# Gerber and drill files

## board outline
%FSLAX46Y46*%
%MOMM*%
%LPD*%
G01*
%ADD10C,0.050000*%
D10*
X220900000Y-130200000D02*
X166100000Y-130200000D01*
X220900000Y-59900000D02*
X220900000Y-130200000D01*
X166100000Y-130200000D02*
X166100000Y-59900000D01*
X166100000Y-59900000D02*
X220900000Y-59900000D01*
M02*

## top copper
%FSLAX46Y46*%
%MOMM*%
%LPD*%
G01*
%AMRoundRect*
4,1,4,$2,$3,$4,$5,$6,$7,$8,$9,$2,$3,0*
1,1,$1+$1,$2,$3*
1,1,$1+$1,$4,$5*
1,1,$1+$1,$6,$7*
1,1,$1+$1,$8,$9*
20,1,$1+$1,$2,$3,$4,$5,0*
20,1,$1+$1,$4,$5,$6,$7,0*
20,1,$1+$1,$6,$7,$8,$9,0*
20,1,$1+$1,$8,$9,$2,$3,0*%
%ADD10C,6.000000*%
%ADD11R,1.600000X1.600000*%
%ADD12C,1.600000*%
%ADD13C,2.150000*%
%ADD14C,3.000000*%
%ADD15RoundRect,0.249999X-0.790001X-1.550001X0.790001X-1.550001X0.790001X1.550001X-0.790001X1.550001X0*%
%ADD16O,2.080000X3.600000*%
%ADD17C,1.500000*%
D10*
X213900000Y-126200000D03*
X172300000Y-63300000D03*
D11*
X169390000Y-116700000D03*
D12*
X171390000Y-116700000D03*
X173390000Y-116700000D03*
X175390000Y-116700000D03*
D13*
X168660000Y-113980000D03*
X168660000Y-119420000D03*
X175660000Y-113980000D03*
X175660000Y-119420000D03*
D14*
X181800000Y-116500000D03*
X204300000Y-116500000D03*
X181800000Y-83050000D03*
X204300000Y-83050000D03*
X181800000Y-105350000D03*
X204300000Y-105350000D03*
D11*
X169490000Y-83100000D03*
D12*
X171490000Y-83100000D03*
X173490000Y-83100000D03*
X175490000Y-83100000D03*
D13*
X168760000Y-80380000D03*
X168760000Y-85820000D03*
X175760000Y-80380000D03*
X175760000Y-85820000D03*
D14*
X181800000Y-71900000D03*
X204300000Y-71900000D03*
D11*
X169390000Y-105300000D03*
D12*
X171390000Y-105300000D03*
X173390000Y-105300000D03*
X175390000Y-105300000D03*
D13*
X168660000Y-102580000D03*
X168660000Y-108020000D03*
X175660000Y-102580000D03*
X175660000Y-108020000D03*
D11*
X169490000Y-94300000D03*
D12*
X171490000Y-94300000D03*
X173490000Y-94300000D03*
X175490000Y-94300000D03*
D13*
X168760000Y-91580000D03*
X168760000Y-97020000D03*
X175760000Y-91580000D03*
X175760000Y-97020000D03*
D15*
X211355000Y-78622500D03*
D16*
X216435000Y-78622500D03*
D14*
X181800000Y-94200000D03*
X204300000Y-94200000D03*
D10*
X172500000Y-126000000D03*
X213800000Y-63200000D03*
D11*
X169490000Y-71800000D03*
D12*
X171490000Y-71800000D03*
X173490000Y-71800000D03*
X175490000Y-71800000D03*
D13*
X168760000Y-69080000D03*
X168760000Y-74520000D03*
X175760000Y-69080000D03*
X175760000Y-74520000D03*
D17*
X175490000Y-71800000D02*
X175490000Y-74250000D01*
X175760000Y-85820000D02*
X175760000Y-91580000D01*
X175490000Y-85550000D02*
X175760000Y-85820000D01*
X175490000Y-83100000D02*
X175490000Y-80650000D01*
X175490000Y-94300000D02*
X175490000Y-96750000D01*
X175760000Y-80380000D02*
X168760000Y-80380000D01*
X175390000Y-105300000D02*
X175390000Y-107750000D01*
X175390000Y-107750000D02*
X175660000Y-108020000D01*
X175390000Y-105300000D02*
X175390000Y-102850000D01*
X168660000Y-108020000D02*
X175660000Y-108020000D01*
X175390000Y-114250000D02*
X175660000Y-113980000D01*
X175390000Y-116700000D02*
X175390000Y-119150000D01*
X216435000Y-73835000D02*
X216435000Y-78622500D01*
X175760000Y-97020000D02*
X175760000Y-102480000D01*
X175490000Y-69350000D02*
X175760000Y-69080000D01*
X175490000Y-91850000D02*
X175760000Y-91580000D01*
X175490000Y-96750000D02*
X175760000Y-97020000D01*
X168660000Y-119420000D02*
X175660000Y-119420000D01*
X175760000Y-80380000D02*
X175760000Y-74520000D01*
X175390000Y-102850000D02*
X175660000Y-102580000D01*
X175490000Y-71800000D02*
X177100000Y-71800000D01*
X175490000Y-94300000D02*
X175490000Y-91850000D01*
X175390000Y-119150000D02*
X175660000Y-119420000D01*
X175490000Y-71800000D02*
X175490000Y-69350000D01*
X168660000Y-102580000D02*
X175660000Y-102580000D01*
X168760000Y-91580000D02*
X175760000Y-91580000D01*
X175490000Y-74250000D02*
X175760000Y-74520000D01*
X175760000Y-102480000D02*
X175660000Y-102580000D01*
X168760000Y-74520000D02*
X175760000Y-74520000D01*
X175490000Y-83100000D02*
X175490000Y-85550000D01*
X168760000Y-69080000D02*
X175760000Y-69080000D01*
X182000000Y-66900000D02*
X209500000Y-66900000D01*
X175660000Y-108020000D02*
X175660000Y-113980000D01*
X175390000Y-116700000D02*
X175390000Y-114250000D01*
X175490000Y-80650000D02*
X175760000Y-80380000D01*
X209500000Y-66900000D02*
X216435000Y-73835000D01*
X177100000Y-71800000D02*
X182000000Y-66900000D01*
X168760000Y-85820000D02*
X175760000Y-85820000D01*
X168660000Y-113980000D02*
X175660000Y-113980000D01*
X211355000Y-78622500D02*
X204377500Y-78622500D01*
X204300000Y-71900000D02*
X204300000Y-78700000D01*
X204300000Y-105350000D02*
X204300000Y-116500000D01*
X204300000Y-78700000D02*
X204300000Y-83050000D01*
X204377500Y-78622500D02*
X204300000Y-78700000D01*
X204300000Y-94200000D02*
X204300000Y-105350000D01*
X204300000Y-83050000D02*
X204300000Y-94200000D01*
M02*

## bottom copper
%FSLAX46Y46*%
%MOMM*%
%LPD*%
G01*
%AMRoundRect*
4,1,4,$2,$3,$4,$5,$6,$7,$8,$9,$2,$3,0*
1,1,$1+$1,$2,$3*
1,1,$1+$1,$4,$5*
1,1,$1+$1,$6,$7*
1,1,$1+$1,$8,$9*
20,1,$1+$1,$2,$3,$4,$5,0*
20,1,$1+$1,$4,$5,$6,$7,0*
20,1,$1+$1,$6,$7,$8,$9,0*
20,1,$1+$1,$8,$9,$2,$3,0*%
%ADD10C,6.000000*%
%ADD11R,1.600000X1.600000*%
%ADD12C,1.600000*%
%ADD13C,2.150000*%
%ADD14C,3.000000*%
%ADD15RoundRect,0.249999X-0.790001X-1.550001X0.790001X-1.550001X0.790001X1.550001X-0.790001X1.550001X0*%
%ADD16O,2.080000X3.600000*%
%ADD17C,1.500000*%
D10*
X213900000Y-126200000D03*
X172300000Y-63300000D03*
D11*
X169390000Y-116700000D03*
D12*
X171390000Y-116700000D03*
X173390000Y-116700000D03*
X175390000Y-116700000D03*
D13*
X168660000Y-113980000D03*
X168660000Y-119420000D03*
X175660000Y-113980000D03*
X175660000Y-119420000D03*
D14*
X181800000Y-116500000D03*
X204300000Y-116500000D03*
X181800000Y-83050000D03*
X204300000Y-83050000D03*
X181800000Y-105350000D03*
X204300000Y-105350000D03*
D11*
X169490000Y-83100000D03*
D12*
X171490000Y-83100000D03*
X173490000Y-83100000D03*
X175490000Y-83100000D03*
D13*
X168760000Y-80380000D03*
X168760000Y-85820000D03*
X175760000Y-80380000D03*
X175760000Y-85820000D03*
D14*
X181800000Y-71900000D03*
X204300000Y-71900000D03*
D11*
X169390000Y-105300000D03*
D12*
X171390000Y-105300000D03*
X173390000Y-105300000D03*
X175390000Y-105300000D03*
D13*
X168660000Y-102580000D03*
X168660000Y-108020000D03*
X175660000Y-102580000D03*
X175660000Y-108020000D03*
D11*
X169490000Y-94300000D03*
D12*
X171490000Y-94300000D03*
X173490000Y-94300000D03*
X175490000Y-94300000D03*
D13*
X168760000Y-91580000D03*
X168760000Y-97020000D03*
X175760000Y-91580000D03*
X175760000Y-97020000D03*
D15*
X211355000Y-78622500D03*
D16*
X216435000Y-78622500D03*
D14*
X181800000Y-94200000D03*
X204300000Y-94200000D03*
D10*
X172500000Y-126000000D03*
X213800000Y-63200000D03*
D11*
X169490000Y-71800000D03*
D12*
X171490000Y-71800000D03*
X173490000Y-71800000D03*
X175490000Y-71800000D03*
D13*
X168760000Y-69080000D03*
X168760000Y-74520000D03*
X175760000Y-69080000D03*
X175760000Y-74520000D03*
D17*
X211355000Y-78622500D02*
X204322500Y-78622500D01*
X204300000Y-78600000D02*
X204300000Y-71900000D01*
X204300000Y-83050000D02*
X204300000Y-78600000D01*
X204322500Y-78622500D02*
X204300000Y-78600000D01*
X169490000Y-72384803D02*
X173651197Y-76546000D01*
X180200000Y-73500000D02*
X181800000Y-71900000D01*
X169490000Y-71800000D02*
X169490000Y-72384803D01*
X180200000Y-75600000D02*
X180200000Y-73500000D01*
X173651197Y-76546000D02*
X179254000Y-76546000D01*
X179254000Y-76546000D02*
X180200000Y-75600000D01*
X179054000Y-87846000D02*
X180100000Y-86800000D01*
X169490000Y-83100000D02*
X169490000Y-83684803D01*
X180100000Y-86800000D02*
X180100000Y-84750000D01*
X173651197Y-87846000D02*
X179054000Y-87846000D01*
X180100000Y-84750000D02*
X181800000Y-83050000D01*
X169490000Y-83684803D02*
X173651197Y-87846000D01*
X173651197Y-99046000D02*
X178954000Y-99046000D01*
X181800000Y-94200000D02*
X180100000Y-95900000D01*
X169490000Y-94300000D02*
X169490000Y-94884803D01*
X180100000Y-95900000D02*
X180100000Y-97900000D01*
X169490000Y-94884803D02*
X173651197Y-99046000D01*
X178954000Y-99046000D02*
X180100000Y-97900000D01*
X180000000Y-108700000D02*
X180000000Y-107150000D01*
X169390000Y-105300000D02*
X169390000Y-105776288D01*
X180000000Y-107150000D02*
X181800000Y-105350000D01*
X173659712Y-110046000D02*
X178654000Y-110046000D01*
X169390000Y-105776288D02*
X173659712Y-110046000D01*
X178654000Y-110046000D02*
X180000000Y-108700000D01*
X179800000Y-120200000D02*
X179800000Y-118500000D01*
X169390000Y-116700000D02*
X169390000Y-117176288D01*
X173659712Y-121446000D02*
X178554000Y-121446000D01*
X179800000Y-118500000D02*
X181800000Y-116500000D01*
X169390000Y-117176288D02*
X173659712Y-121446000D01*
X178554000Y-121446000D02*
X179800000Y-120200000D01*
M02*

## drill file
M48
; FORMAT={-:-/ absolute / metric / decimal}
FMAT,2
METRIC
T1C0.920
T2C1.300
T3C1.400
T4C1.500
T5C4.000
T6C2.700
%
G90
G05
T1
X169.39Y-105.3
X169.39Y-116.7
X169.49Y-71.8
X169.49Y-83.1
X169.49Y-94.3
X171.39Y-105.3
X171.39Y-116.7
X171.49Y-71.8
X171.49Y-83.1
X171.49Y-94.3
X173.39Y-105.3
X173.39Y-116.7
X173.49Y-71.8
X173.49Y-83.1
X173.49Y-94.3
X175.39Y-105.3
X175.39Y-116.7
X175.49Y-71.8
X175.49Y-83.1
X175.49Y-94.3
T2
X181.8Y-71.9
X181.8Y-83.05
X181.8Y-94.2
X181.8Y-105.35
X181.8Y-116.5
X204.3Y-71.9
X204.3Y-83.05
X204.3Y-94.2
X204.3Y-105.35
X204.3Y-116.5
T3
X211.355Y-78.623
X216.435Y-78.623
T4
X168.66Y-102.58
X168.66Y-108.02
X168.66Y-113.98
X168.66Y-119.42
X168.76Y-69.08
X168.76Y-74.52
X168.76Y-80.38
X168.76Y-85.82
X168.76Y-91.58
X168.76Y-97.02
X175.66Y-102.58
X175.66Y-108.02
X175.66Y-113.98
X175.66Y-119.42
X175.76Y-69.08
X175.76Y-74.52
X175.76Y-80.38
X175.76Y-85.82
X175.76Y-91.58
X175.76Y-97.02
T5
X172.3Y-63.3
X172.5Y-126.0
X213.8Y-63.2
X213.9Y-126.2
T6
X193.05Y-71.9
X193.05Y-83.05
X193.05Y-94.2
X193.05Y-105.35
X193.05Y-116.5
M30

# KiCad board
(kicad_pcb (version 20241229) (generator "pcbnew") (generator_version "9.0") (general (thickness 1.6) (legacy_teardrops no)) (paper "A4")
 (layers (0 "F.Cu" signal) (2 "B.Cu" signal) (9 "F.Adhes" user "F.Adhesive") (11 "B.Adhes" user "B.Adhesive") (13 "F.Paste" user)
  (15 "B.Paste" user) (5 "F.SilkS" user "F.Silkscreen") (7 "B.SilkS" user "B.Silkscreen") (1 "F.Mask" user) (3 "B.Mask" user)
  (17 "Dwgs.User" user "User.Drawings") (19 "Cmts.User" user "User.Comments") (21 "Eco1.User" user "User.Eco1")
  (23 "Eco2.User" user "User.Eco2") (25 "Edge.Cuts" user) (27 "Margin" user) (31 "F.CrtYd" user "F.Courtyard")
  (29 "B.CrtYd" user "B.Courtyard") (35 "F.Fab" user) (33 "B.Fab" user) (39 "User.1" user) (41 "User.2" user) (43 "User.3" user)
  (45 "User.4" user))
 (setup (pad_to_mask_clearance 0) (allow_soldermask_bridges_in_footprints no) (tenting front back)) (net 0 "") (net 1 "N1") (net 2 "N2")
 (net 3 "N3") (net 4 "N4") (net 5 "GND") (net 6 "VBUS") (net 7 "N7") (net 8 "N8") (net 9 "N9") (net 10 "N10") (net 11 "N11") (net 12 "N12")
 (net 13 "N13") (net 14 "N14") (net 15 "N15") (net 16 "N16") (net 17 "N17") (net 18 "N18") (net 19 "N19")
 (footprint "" (layer "F.Cu") (at 213.9 126.2)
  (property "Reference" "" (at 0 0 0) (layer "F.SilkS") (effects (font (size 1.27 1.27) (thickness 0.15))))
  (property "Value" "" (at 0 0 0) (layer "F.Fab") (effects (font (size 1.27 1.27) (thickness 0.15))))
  (pad "1" thru_hole circle (at 0 0) (size 6 6) (drill 4) (layers "*.Cu" "*.Mask") (remove_unused_layers no) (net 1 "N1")))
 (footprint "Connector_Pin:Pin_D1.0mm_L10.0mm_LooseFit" (layer "F.Cu") (at 172.3 63.3)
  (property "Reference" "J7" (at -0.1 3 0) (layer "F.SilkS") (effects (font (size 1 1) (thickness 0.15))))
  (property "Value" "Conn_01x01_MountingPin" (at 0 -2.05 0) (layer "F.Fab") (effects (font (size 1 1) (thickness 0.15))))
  (pad "1" thru_hole circle (at 0 0) (size 6 6) (drill 4) (layers "*.Cu" "*.Mask") (remove_unused_layers no) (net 1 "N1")))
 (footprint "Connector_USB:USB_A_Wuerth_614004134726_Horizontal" (layer "F.Cu") (at 169.39 116.7)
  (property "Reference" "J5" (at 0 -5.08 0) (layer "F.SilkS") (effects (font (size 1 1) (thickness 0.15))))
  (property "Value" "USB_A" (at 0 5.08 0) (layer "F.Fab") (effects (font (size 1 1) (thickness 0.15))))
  (pad "1" thru_hole rect (at 0 0) (size 1.6 1.6) (drill 0.92) (layers "*.Cu" "*.Mask") (remove_unused_layers no) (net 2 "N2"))
  (pad "2" thru_hole circle (at 2 0) (size 1.6 1.6) (drill 0.92) (layers "*.Cu" "*.Mask") (remove_unused_layers no) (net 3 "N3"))
  (pad "3" thru_hole circle (at 4 0) (size 1.6 1.6) (drill 0.92) (layers "*.Cu" "*.Mask") (remove_unused_layers no) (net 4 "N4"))
  (pad "4" thru_hole circle (at 6 0) (size 1.6 1.6) (drill 0.92) (layers "*.Cu" "*.Mask") (remove_unused_layers no) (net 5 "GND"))
  (pad "5" thru_hole circle (at -0.73 -2.72) (size 2.15 2.15) (drill 1.5) (layers "*.Cu" "*.Mask") (remove_unused_layers no) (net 5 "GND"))
  (pad "5" thru_hole circle (at -0.73 2.72) (size 2.15 2.15) (drill 1.5) (layers "*.Cu" "*.Mask") (remove_unused_layers no) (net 5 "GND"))
  (pad "5" thru_hole circle (at 6.27 -2.72) (size 2.15 2.15) (drill 1.5) (layers "*.Cu" "*.Mask") (remove_unused_layers no) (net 5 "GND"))
  (pad "5" thru_hole circle (at 6.27 2.72) (size 2.15 2.15) (drill 1.5) (layers "*.Cu" "*.Mask") (remove_unused_layers no) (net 5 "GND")))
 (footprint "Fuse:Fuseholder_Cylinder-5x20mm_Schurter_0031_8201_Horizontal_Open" (layer "F.Cu") (at 181.8 116.5)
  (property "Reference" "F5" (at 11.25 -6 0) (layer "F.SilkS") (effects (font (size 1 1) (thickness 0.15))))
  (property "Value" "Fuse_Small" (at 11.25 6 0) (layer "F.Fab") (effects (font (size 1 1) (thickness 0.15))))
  (pad "" np_thru_hole circle (at 11.25 0) (size 2.7 2.7) (drill 2.7) (layers "*.Cu" "*.Mask"))
  (pad "1" thru_hole circle (at 0 0) (size 3 3) (drill 1.3) (layers "*.Cu" "*.Mask") (remove_unused_layers no) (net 2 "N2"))
  (pad "2" thru_hole circle (at 22.5 0) (size 3 3) (drill 1.3) (layers "*.Cu" "*.Mask") (remove_unused_layers no) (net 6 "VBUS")))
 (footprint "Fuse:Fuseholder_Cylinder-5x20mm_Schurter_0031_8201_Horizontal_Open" (layer "F.Cu") (at 181.8 83.05)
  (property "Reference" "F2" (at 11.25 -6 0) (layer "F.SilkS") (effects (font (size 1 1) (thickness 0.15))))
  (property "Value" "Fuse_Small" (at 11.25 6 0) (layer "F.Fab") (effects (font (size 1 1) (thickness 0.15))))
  (pad "" np_thru_hole circle (at 11.25 0) (size 2.7 2.7) (drill 2.7) (layers "*.Cu" "*.Mask"))
  (pad "1" thru_hole circle (at 0 0) (size 3 3) (drill 1.3) (layers "*.Cu" "*.Mask") (remove_unused_layers no) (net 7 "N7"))
  (pad "2" thru_hole circle (at 22.5 0) (size 3 3) (drill 1.3) (layers "*.Cu" "*.Mask") (remove_unused_layers no) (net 6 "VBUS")))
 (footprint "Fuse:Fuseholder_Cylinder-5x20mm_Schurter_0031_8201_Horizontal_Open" (layer "F.Cu") (at 181.8 105.35)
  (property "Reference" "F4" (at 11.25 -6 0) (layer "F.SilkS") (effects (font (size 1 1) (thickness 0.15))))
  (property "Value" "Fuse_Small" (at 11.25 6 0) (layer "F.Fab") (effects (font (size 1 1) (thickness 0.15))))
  (pad "" np_thru_hole circle (at 11.25 0) (size 2.7 2.7) (drill 2.7) (layers "*.Cu" "*.Mask"))
  (pad "1" thru_hole circle (at 0 0) (size 3 3) (drill 1.3) (layers "*.Cu" "*.Mask") (remove_unused_layers no) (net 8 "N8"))
  (pad "2" thru_hole circle (at 22.5 0) (size 3 3) (drill 1.3) (layers "*.Cu" "*.Mask") (remove_unused_layers no) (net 6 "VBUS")))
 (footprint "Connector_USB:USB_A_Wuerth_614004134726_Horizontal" (layer "F.Cu") (at 169.49 83.1)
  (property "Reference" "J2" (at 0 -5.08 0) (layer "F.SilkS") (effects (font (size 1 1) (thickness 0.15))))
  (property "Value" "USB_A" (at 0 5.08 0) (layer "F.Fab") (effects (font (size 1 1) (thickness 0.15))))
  (pad "1" thru_hole rect (at 0 0) (size 1.6 1.6) (drill 0.92) (layers "*.Cu" "*.Mask") (remove_unused_layers no) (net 7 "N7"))
  (pad "2" thru_hole circle (at 2 0) (size 1.6 1.6) (drill 0.92) (layers "*.Cu" "*.Mask") (remove_unused_layers no) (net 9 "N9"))
  (pad "3" thru_hole circle (at 4 0) (size 1.6 1.6) (drill 0.92) (layers "*.Cu" "*.Mask") (remove_unused_layers no) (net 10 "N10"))
  (pad "4" thru_hole circle (at 6 0) (size 1.6 1.6) (drill 0.92) (layers "*.Cu" "*.Mask") (remove_unused_layers no) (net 5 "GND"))
  (pad "5" thru_hole circle (at -0.73 -2.72) (size 2.15 2.15) (drill 1.5) (layers "*.Cu" "*.Mask") (remove_unused_layers no) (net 5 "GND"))
  (pad "5" thru_hole circle (at -0.73 2.72) (size 2.15 2.15) (drill 1.5) (layers "*.Cu" "*.Mask") (remove_unused_layers no) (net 5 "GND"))
  (pad "5" thru_hole circle (at 6.27 -2.72) (size 2.15 2.15) (drill 1.5) (layers "*.Cu" "*.Mask") (remove_unused_layers no) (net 5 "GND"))
  (pad "5" thru_hole circle (at 6.27 2.72) (size 2.15 2.15) (drill 1.5) (layers "*.Cu" "*.Mask") (remove_unused_layers no) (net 5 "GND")))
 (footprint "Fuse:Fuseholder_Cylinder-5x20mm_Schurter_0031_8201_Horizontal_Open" (layer "F.Cu") (at 181.8 71.9)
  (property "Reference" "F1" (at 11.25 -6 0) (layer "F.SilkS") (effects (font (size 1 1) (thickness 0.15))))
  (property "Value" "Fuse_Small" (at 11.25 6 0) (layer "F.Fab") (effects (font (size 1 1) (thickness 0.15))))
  (pad "" np_thru_hole circle (at 11.25 0) (size 2.7 2.7) (drill 2.7) (layers "*.Cu" "*.Mask"))
  (pad "1" thru_hole circle (at 0 0) (size 3 3) (drill 1.3) (layers "*.Cu" "*.Mask") (remove_unused_layers no) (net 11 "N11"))
  (pad "2" thru_hole circle (at 22.5 0) (size 3 3) (drill 1.3) (layers "*.Cu" "*.Mask") (remove_unused_layers no) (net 6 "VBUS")))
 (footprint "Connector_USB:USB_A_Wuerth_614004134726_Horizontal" (layer "F.Cu") (at 169.39 105.3)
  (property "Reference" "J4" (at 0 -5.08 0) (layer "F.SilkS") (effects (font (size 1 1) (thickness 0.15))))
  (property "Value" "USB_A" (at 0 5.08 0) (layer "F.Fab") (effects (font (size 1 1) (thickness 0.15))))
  (pad "1" thru_hole rect (at 0 0) (size 1.6 1.6) (drill 0.92) (layers "*.Cu" "*.Mask") (remove_unused_layers no) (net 8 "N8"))
  (pad "2" thru_hole circle (at 2 0) (size 1.6 1.6) (drill 0.92) (layers "*.Cu" "*.Mask") (remove_unused_layers no) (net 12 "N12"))
  (pad "3" thru_hole circle (at 4 0) (size 1.6 1.6) (drill 0.92) (layers "*.Cu" "*.Mask") (remove_unused_layers no) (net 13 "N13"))
  (pad "4" thru_hole circle (at 6 0) (size 1.6 1.6) (drill 0.92) (layers "*.Cu" "*.Mask") (remove_unused_layers no) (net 5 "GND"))
  (pad "5" thru_hole circle (at -0.73 -2.72) (size 2.15 2.15) (drill 1.5) (layers "*.Cu" "*.Mask") (remove_unused_layers no) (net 5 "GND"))
  (pad "5" thru_hole circle (at -0.73 2.72) (size 2.15 2.15) (drill 1.5) (layers "*.Cu" "*.Mask") (remove_unused_layers no) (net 5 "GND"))
  (pad "5" thru_hole circle (at 6.27 -2.72) (size 2.15 2.15) (drill 1.5) (layers "*.Cu" "*.Mask") (remove_unused_layers no) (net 5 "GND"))
  (pad "5" thru_hole circle (at 6.27 2.72) (size 2.15 2.15) (drill 1.5) (layers "*.Cu" "*.Mask") (remove_unused_layers no) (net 5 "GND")))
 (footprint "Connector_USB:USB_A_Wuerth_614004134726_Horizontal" (layer "F.Cu") (at 169.49 94.3)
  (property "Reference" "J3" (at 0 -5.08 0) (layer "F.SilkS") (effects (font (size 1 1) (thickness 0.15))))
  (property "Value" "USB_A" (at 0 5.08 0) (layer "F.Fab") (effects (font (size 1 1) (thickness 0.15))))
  (pad "1" thru_hole rect (at 0 0) (size 1.6 1.6) (drill 0.92) (layers "*.Cu" "*.Mask") (remove_unused_layers no) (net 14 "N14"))
  (pad "2" thru_hole circle (at 2 0) (size 1.6 1.6) (drill 0.92) (layers "*.Cu" "*.Mask") (remove_unused_layers no) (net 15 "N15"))
  (pad "3" thru_hole circle (at 4 0) (size 1.6 1.6) (drill 0.92) (layers "*.Cu" "*.Mask") (remove_unused_layers no) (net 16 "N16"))
  (pad "4" thru_hole circle (at 6 0) (size 1.6 1.6) (drill 0.92) (layers "*.Cu" "*.Mask") (remove_unused_layers no) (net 5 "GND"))
  (pad "5" thru_hole circle (at -0.73 -2.72) (size 2.15 2.15) (drill 1.5) (layers "*.Cu" "*.Mask") (remove_unused_layers no) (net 5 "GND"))
  (pad "5" thru_hole circle (at -0.73 2.72) (size 2.15 2.15) (drill 1.5) (layers "*.Cu" "*.Mask") (remove_unused_layers no) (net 5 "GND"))
  (pad "5" thru_hole circle (at 6.27 -2.72) (size 2.15 2.15) (drill 1.5) (layers "*.Cu" "*.Mask") (remove_unused_layers no) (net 5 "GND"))
  (pad "5" thru_hole circle (at 6.27 2.72) (size 2.15 2.15) (drill 1.5) (layers "*.Cu" "*.Mask") (remove_unused_layers no) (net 5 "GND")))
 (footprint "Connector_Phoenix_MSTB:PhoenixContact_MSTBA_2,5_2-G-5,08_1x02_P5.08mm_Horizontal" (layer "F.Cu") (at 211.355 78.6225)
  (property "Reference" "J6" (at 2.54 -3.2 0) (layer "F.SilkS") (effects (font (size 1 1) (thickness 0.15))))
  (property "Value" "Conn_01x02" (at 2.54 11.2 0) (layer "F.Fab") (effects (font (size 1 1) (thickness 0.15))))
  (pad "1" thru_hole roundrect (at 0 0) (size 2.08 3.6) (drill 1.4) (layers "*.Cu" "*.Mask") (remove_unused_layers no)
   (roundrect_rratio 0.120192) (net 6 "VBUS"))
  (pad "2" thru_hole oval (at 5.08 0) (size 2.08 3.6) (drill 1.4) (layers "*.Cu" "*.Mask") (remove_unused_layers no) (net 5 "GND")))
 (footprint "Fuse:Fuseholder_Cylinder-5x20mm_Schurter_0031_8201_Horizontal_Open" (layer "F.Cu") (at 181.8 94.2)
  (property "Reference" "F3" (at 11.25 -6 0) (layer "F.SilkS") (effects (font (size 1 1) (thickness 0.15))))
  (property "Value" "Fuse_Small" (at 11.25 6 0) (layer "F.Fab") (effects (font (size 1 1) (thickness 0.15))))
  (pad "" np_thru_hole circle (at 11.25 0) (size 2.7 2.7) (drill 2.7) (layers "*.Cu" "*.Mask"))
  (pad "1" thru_hole circle (at 0 0) (size 3 3) (drill 1.3) (layers "*.Cu" "*.Mask") (remove_unused_layers no) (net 14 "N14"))
  (pad "2" thru_hole circle (at 22.5 0) (size 3 3) (drill 1.3) (layers "*.Cu" "*.Mask") (remove_unused_layers no) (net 6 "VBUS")))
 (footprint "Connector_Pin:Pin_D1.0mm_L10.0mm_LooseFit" (layer "F.Cu") (at 172.5 126)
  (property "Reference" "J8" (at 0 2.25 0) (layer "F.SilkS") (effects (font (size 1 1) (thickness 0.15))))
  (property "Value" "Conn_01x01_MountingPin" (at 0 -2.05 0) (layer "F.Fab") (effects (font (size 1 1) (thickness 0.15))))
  (pad "1" thru_hole circle (at 0 0) (size 6 6) (drill 4) (layers "*.Cu" "*.Mask") (remove_unused_layers no) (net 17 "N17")))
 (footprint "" (layer "F.Cu") (at 213.8 63.2)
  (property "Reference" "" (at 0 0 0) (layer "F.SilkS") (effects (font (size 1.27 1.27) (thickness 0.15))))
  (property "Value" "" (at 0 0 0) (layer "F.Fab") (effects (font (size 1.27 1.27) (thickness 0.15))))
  (pad "1" thru_hole circle (at 0 0) (size 6 6) (drill 4) (layers "*.Cu" "*.Mask") (remove_unused_layers no) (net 1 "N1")))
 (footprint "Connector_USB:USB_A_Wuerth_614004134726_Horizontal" (layer "F.Cu") (at 169.49 71.8)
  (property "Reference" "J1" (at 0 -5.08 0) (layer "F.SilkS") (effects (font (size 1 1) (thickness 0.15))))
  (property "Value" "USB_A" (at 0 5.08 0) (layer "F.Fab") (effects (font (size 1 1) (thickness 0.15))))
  (pad "1" thru_hole rect (at 0 0) (size 1.6 1.6) (drill 0.92) (layers "*.Cu" "*.Mask") (remove_unused_layers no) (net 11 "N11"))
  (pad "2" thru_hole circle (at 2 0) (size 1.6 1.6) (drill 0.92) (layers "*.Cu" "*.Mask") (remove_unused_layers no) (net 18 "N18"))
  (pad "3" thru_hole circle (at 4 0) (size 1.6 1.6) (drill 0.92) (layers "*.Cu" "*.Mask") (remove_unused_layers no) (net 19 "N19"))
  (pad "4" thru_hole circle (at 6 0) (size 1.6 1.6) (drill 0.92) (layers "*.Cu" "*.Mask") (remove_unused_layers no) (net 5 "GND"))
  (pad "5" thru_hole circle (at -0.73 -2.72) (size 2.15 2.15) (drill 1.5) (layers "*.Cu" "*.Mask") (remove_unused_layers no) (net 5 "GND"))
  (pad "5" thru_hole circle (at -0.73 2.72) (size 2.15 2.15) (drill 1.5) (layers "*.Cu" "*.Mask") (remove_unused_layers no) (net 5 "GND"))
  (pad "5" thru_hole circle (at 6.27 -2.72) (size 2.15 2.15) (drill 1.5) (layers "*.Cu" "*.Mask") (remove_unused_layers no) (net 5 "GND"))
  (pad "5" thru_hole circle (at 6.27 2.72) (size 2.15 2.15) (drill 1.5) (layers "*.Cu" "*.Mask") (remove_unused_layers no) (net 5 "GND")))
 (gr_line (start 220.9 130.2) (end 166.1 130.2) (stroke (width 0.05) (type default)) (layer "Edge.Cuts"))
 (gr_line (start 220.9 59.9) (end 220.9 130.2) (stroke (width 0.05) (type default)) (layer "Edge.Cuts"))
 (gr_line (start 166.1 130.2) (end 166.1 59.9) (stroke (width 0.05) (type default)) (layer "Edge.Cuts"))
 (gr_line (start 166.1 59.9) (end 220.9 59.9) (stroke (width 0.05) (type default)) (layer "Edge.Cuts"))
 (segment (start 175.49 71.8) (end 175.49 74.25) (width 1.5) (layer "F.Cu") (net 5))
 (segment (start 175.76 85.82) (end 175.76 91.58) (width 1.5) (layer "F.Cu") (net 5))
 (segment (start 175.49 85.55) (end 175.76 85.82) (width 1.5) (layer "F.Cu") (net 5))
 (segment (start 175.49 83.1) (end 175.49 80.65) (width 1.5) (layer "F.Cu") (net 5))
 (segment (start 175.49 94.3) (end 175.49 96.75) (width 1.5) (layer "F.Cu") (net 5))
 (segment (start 175.76 80.38) (end 168.76 80.38) (width 1.5) (layer "F.Cu") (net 5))
 (segment (start 175.39 105.3) (end 175.39 107.75) (width 1.5) (layer "F.Cu") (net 5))
 (segment (start 175.39 107.75) (end 175.66 108.02) (width 1.5) (layer "F.Cu") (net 5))
 (segment (start 175.39 105.3) (end 175.39 102.85) (width 1.5) (layer "F.Cu") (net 5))
 (segment (start 168.66 108.02) (end 175.66 108.02) (width 1.5) (layer "F.Cu") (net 5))
 (segment (start 175.39 114.25) (end 175.66 113.98) (width 1.5) (layer "F.Cu") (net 5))
 (segment (start 175.39 116.7) (end 175.39 119.15) (width 1.5) (layer "F.Cu") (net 5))
 (segment (start 216.435 73.835) (end 216.435 78.6225) (width 1.5) (layer "F.Cu") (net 5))
 (segment (start 175.76 97.02) (end 175.76 102.48) (width 1.5) (layer "F.Cu") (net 5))
 (segment (start 175.49 69.35) (end 175.76 69.08) (width 1.5) (layer "F.Cu") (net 5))
 (segment (start 175.49 91.85) (end 175.76 91.58) (width 1.5) (layer "F.Cu") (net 5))
 (segment (start 175.49 96.75) (end 175.76 97.02) (width 1.5) (layer "F.Cu") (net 5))
 (segment (start 168.66 119.42) (end 175.66 119.42) (width 1.5) (layer "F.Cu") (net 5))
 (segment (start 175.76 80.38) (end 175.76 74.52) (width 1.5) (layer "F.Cu") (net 5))
 (segment (start 175.39 102.85) (end 175.66 102.58) (width 1.5) (layer "F.Cu") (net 5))
 (segment (start 175.49 71.8) (end 177.1 71.8) (width 1.5) (layer "F.Cu") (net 5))
 (segment (start 175.49 94.3) (end 175.49 91.85) (width 1.5) (layer "F.Cu") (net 5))
 (segment (start 175.39 119.15) (end 175.66 119.42) (width 1.5) (layer "F.Cu") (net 5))
 (segment (start 175.49 71.8) (end 175.49 69.35) (width 1.5) (layer "F.Cu") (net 5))
 (segment (start 168.66 102.58) (end 175.66 102.58) (width 1.5) (layer "F.Cu") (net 5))
 (segment (start 168.76 91.58) (end 175.76 91.58) (width 1.5) (layer "F.Cu") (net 5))
 (segment (start 175.49 74.25) (end 175.76 74.52) (width 1.5) (layer "F.Cu") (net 5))
 (segment (start 175.76 102.48) (end 175.66 102.58) (width 1.5) (layer "F.Cu") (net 5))
 (segment (start 168.76 74.52) (end 175.76 74.52) (width 1.5) (layer "F.Cu") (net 5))
 (segment (start 175.49 83.1) (end 175.49 85.55) (width 1.5) (layer "F.Cu") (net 5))
 (segment (start 168.76 69.08) (end 175.76 69.08) (width 1.5) (layer "F.Cu") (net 5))
 (segment (start 182 66.9) (end 209.5 66.9) (width 1.5) (layer "F.Cu") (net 5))
 (segment (start 175.66 108.02) (end 175.66 113.98) (width 1.5) (layer "F.Cu") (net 5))
 (segment (start 175.39 116.7) (end 175.39 114.25) (width 1.5) (layer "F.Cu") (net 5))
 (segment (start 175.49 80.65) (end 175.76 80.38) (width 1.5) (layer "F.Cu") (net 5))
 (segment (start 209.5 66.9) (end 216.435 73.835) (width 1.5) (layer "F.Cu") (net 5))
 (segment (start 177.1 71.8) (end 182 66.9) (width 1.5) (layer "F.Cu") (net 5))
 (segment (start 168.76 85.82) (end 175.76 85.82) (width 1.5) (layer "F.Cu") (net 5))
 (segment (start 168.66 113.98) (end 175.66 113.98) (width 1.5) (layer "F.Cu") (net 5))
 (segment (start 211.355 78.6225) (end 204.3775 78.6225) (width 1.5) (layer "F.Cu") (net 6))
 (segment (start 204.3 71.9) (end 204.3 78.7) (width 1.5) (layer "F.Cu") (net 6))
 (segment (start 204.3 105.35) (end 204.3 116.5) (width 1.5) (layer "F.Cu") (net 6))
 (segment (start 204.3 78.7) (end 204.3 83.05) (width 1.5) (layer "F.Cu") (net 6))
 (segment (start 204.3775 78.6225) (end 204.3 78.7) (width 1.5) (layer "F.Cu") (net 6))
 (segment (start 204.3 94.2) (end 204.3 105.35) (width 1.5) (layer "F.Cu") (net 6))
 (segment (start 204.3 83.05) (end 204.3 94.2) (width 1.5) (layer "F.Cu") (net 6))
 (segment (start 211.355 78.6225) (end 204.3225 78.6225) (width 1.5) (layer "B.Cu") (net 6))
 (segment (start 204.3 78.6) (end 204.3 71.9) (width 1.5) (layer "B.Cu") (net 6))
 (segment (start 204.3 83.05) (end 204.3 78.6) (width 1.5) (layer "B.Cu") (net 6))
 (segment (start 204.3225 78.6225) (end 204.3 78.6) (width 1.5) (layer "B.Cu") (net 6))
 (segment (start 169.49 72.384803) (end 173.651197 76.546) (width 1.5) (layer "B.Cu") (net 11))
 (segment (start 180.2 73.5) (end 181.8 71.9) (width 1.5) (layer "B.Cu") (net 11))
 (segment (start 169.49 71.8) (end 169.49 72.384803) (width 1.5) (layer "B.Cu") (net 11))
 (segment (start 180.2 75.6) (end 180.2 73.5) (width 1.5) (layer "B.Cu") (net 11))
 (segment (start 173.651197 76.546) (end 179.254 76.546) (width 1.5) (layer "B.Cu") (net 11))
 (segment (start 179.254 76.546) (end 180.2 75.6) (width 1.5) (layer "B.Cu") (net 11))
 (segment (start 179.054 87.846) (end 180.1 86.8) (width 1.5) (layer "B.Cu") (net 7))
 (segment (start 169.49 83.1) (end 169.49 83.684803) (width 1.5) (layer "B.Cu") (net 7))
 (segment (start 180.1 86.8) (end 180.1 84.75) (width 1.5) (layer "B.Cu") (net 7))
 (segment (start 173.651197 87.846) (end 179.054 87.846) (width 1.5) (layer "B.Cu") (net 7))
 (segment (start 180.1 84.75) (end 181.8 83.05) (width 1.5) (layer "B.Cu") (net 7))
 (segment (start 169.49 83.684803) (end 173.651197 87.846) (width 1.5) (layer "B.Cu") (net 7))
 (segment (start 173.651197 99.046) (end 178.954 99.046) (width 1.5) (layer "B.Cu") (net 14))
 (segment (start 181.8 94.2) (end 180.1 95.9) (width 1.5) (layer "B.Cu") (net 14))
 (segment (start 169.49 94.3) (end 169.49 94.884803) (width 1.5) (layer "B.Cu") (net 14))
 (segment (start 180.1 95.9) (end 180.1 97.9) (width 1.5) (layer "B.Cu") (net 14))
 (segment (start 169.49 94.884803) (end 173.651197 99.046) (width 1.5) (layer "B.Cu") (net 14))
 (segment (start 178.954 99.046) (end 180.1 97.9) (width 1.5) (layer "B.Cu") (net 14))
 (segment (start 180 108.7) (end 180 107.15) (width 1.5) (layer "B.Cu") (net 8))
 (segment (start 169.39 105.3) (end 169.39 105.776288) (width 1.5) (layer "B.Cu") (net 8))
 (segment (start 180 107.15) (end 181.8 105.35) (width 1.5) (layer "B.Cu") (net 8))
 (segment (start 173.659712 110.046) (end 178.654 110.046) (width 1.5) (layer "B.Cu") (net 8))
 (segment (start 169.39 105.776288) (end 173.659712 110.046) (width 1.5) (layer "B.Cu") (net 8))
 (segment (start 178.654 110.046) (end 180 108.7) (width 1.5) (layer "B.Cu") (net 8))
 (segment (start 179.8 120.2) (end 179.8 118.5) (width 1.5) (layer "B.Cu") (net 2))
 (segment (start 169.39 116.7) (end 169.39 117.176288) (width 1.5) (layer "B.Cu") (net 2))
 (segment (start 173.659712 121.446) (end 178.554 121.446) (width 1.5) (layer "B.Cu") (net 2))
 (segment (start 179.8 118.5) (end 181.8 116.5) (width 1.5) (layer "B.Cu") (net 2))
 (segment (start 169.39 117.176288) (end 173.659712 121.446) (width 1.5) (layer "B.Cu") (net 2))
 (segment (start 178.554 121.446) (end 179.8 120.2) (width 1.5) (layer "B.Cu") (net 2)))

